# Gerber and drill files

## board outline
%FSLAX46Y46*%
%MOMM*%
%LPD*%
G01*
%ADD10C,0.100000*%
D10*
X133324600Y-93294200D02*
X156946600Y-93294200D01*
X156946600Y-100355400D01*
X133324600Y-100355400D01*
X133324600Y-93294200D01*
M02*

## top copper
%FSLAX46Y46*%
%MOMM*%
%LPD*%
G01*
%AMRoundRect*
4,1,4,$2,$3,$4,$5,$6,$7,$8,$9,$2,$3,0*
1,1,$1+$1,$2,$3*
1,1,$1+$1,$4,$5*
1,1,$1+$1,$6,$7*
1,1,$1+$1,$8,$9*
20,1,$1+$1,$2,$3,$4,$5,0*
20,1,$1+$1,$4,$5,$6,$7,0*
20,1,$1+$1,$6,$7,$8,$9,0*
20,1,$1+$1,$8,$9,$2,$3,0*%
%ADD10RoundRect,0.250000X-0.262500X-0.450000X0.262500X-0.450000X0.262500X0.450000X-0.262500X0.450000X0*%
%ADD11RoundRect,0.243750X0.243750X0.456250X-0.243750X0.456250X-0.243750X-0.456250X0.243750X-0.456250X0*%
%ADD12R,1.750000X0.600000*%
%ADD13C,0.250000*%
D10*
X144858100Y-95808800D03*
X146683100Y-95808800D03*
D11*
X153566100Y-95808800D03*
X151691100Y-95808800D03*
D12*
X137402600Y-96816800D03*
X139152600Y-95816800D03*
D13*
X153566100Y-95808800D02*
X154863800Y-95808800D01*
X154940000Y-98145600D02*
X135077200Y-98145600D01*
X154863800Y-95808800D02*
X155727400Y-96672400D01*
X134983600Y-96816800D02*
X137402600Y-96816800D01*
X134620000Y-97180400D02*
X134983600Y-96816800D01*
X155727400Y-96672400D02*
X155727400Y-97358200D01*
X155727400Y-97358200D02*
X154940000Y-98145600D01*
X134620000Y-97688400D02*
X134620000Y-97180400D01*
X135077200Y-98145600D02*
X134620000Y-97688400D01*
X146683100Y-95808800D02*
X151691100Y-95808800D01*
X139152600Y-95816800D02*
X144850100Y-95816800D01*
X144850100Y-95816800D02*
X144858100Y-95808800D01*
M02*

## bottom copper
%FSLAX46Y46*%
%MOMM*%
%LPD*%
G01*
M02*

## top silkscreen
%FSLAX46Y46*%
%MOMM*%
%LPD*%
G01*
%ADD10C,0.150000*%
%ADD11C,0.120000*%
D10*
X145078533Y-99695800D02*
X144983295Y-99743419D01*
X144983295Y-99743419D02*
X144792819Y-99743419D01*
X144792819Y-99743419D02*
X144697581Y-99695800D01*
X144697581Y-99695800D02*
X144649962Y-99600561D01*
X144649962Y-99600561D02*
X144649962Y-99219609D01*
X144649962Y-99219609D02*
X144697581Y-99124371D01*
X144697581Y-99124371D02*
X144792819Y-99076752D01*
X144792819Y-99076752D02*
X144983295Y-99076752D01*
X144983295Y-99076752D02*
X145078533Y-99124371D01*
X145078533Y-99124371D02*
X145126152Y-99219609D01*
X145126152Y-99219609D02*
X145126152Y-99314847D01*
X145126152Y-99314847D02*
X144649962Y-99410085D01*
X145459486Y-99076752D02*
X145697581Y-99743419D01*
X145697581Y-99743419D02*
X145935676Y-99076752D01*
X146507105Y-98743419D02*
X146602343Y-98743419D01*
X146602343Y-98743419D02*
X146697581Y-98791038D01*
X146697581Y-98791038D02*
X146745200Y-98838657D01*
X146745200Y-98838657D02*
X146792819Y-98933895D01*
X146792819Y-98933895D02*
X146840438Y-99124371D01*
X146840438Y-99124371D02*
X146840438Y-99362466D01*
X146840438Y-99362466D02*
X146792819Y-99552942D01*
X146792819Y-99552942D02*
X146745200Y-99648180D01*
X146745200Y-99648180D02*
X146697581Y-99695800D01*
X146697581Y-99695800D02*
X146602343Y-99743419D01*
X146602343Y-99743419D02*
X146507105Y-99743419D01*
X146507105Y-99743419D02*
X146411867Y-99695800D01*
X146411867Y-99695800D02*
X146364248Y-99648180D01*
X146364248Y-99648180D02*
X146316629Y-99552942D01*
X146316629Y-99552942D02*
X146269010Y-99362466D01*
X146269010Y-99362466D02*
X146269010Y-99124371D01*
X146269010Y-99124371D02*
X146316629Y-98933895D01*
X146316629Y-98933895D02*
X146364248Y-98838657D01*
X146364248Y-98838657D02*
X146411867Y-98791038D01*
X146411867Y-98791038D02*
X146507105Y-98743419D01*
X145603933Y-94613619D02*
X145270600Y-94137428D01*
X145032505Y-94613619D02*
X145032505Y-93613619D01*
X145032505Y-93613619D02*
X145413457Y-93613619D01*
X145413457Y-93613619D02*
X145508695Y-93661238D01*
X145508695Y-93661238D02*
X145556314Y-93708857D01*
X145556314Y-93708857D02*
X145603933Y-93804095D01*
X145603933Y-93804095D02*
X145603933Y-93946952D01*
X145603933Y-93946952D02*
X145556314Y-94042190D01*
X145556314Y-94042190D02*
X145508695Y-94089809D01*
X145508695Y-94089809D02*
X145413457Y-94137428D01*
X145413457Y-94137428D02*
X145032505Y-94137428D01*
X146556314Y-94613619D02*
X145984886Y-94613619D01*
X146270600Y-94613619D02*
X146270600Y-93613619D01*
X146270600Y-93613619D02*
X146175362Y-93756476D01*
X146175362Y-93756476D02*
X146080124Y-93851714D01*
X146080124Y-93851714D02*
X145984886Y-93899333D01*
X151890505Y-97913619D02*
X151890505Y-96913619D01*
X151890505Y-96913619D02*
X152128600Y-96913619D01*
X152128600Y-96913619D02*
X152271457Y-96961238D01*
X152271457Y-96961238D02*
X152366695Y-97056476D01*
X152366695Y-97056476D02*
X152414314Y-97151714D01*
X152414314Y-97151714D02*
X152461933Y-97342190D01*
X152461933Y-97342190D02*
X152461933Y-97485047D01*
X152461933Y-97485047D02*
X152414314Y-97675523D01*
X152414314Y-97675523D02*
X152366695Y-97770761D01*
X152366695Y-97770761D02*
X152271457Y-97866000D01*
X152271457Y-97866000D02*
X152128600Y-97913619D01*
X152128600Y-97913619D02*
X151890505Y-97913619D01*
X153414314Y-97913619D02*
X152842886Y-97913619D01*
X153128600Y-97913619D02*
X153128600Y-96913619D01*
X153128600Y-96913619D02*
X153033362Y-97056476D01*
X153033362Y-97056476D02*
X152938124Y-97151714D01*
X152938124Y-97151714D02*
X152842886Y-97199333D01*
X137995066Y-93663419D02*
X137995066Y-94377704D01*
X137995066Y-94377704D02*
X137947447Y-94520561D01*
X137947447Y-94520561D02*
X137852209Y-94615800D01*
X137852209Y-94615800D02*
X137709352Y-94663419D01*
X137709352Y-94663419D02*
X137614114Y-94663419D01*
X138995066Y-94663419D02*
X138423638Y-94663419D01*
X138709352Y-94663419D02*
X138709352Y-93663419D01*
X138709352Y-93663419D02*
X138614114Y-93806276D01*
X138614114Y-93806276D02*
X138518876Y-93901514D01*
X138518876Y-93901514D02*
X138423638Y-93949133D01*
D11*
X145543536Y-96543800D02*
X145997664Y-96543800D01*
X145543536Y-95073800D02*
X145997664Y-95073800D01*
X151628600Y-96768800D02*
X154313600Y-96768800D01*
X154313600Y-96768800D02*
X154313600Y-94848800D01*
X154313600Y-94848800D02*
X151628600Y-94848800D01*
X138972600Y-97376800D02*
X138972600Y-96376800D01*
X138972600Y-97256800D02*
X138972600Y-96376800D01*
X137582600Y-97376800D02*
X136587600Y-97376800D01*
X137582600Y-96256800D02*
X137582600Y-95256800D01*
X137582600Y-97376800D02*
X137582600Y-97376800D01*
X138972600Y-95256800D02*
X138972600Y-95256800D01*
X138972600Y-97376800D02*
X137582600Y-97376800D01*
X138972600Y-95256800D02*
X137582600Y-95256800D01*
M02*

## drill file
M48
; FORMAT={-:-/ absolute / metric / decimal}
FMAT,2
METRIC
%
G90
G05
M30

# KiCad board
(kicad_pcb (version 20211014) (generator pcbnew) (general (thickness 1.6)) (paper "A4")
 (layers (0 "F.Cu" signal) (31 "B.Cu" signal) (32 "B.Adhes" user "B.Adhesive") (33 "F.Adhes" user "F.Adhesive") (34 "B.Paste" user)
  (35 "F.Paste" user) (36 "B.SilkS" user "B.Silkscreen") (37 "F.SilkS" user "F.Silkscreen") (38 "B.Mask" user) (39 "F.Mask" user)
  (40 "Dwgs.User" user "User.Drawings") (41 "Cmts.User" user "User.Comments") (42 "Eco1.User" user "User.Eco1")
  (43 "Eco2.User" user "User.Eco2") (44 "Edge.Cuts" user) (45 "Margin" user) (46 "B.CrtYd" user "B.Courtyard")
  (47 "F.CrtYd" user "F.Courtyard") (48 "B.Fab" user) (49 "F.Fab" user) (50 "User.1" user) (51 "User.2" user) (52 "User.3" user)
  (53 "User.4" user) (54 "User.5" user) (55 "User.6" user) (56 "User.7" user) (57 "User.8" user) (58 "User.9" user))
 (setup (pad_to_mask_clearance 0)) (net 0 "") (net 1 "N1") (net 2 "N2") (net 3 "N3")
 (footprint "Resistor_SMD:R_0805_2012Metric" (layer "F.Cu") (at 145.7706 95.8088)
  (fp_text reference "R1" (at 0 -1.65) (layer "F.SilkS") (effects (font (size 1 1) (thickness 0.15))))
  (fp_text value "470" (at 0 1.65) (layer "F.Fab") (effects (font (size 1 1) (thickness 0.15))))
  (fp_line (start -0.227064 0.735) (end 0.227064 0.735) (layer "F.SilkS") (width 0.12))
  (fp_line (start -0.227064 -0.735) (end 0.227064 -0.735) (layer "F.SilkS") (width 0.12))
  (pad "1" smd roundrect (at -0.9125 0) (size 1.025 1.4) (layers "F.Cu" "F.Paste" "F.Mask") (roundrect_rratio 0.243902) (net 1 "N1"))
  (pad "2" smd roundrect (at 0.9125 0) (size 1.025 1.4) (layers "F.Cu" "F.Paste" "F.Mask") (roundrect_rratio 0.243902) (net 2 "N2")))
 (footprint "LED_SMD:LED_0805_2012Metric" (layer "F.Cu") (at 152.6286 95.8088 180)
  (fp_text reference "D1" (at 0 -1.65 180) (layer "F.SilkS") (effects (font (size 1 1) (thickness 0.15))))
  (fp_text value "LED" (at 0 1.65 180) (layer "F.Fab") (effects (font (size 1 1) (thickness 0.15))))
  (fp_line (start 1 -0.96) (end -1.685 -0.96) (layer "F.SilkS") (width 0.12))
  (fp_line (start -1.685 -0.96) (end -1.685 0.96) (layer "F.SilkS") (width 0.12))
  (fp_line (start -1.685 0.96) (end 1 0.96) (layer "F.SilkS") (width 0.12))
  (pad "1" smd roundrect (at -0.9375 0 180) (size 0.975 1.4) (layers "F.Cu" "F.Paste" "F.Mask") (roundrect_rratio 0.25) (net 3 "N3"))
  (pad "2" smd roundrect (at 0.9375 0 180) (size 0.975 1.4) (layers "F.Cu" "F.Paste" "F.Mask") (roundrect_rratio 0.25) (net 2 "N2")))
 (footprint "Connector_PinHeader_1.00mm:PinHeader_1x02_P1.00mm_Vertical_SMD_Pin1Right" (layer "F.Cu") (at 138.2776 96.3168 180)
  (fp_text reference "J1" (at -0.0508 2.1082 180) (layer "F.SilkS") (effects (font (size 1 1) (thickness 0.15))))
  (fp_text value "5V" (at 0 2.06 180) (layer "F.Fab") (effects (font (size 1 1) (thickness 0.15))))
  (fp_line (start -0.695 -1.06) (end -0.695 -0.06) (layer "F.SilkS") (width 0.12))
  (fp_line (start -0.695 -0.94) (end -0.695 -0.06) (layer "F.SilkS") (width 0.12))
  (fp_line (start 0.695 -1.06) (end 1.69 -1.06) (layer "F.SilkS") (width 0.12))
  (fp_line (start 0.695 0.06) (end 0.695 1.06) (layer "F.SilkS") (width 0.12))
  (fp_line (start 0.695 -1.06) (end 0.695 -1.06) (layer "F.SilkS") (width 0.12))
  (fp_line (start -0.695 1.06) (end -0.695 1.06) (layer "F.SilkS") (width 0.12))
  (fp_line (start -0.695 -1.06) (end 0.695 -1.06) (layer "F.SilkS") (width 0.12))
  (fp_line (start -0.695 1.06) (end 0.695 1.06) (layer "F.SilkS") (width 0.12))
  (pad "1" smd rect (at 0.875 -0.5 180) (size 1.75 0.6) (layers "F.Cu" "F.Paste" "F.Mask") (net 3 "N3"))
  (pad "2" smd rect (at -0.875 0.5 180) (size 1.75 0.6) (layers "F.Cu" "F.Paste" "F.Mask") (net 1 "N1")))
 (gr_rect (start 133.3246 93.2942) (end 156.9466 100.3554) (layer "Edge.Cuts") (width 0.1) (fill none))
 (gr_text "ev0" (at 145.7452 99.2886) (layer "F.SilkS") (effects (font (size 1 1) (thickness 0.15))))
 (segment (start 153.5661 95.8088) (end 154.8638 95.8088) (width 0.25) (layer "F.Cu") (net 3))
 (segment (start 154.94 98.1456) (end 135.0772 98.1456) (width 0.25) (layer "F.Cu") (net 3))
 (segment (start 154.8638 95.8088) (end 155.7274 96.6724) (width 0.25) (layer "F.Cu") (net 3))
 (segment (start 134.9836 96.8168) (end 137.4026 96.8168) (width 0.25) (layer "F.Cu") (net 3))
 (segment (start 134.62 97.1804) (end 134.9836 96.8168) (width 0.25) (layer "F.Cu") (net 3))
 (segment (start 155.7274 96.6724) (end 155.7274 97.3582) (width 0.25) (layer "F.Cu") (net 3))
 (segment (start 155.7274 97.3582) (end 154.94 98.1456) (width 0.25) (layer "F.Cu") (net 3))
 (segment (start 134.62 97.6884) (end 134.62 97.1804) (width 0.25) (layer "F.Cu") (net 3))
 (segment (start 135.0772 98.1456) (end 134.62 97.6884) (width 0.25) (layer "F.Cu") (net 3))
 (segment (start 146.6831 95.8088) (end 151.6911 95.8088) (width 0.25) (layer "F.Cu") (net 2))
 (segment (start 139.1526 95.8168) (end 144.8501 95.8168) (width 0.25) (layer "F.Cu") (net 1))
 (segment (start 144.8501 95.8168) (end 144.8581 95.8088) (width 0.25) (layer "F.Cu") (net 1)))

